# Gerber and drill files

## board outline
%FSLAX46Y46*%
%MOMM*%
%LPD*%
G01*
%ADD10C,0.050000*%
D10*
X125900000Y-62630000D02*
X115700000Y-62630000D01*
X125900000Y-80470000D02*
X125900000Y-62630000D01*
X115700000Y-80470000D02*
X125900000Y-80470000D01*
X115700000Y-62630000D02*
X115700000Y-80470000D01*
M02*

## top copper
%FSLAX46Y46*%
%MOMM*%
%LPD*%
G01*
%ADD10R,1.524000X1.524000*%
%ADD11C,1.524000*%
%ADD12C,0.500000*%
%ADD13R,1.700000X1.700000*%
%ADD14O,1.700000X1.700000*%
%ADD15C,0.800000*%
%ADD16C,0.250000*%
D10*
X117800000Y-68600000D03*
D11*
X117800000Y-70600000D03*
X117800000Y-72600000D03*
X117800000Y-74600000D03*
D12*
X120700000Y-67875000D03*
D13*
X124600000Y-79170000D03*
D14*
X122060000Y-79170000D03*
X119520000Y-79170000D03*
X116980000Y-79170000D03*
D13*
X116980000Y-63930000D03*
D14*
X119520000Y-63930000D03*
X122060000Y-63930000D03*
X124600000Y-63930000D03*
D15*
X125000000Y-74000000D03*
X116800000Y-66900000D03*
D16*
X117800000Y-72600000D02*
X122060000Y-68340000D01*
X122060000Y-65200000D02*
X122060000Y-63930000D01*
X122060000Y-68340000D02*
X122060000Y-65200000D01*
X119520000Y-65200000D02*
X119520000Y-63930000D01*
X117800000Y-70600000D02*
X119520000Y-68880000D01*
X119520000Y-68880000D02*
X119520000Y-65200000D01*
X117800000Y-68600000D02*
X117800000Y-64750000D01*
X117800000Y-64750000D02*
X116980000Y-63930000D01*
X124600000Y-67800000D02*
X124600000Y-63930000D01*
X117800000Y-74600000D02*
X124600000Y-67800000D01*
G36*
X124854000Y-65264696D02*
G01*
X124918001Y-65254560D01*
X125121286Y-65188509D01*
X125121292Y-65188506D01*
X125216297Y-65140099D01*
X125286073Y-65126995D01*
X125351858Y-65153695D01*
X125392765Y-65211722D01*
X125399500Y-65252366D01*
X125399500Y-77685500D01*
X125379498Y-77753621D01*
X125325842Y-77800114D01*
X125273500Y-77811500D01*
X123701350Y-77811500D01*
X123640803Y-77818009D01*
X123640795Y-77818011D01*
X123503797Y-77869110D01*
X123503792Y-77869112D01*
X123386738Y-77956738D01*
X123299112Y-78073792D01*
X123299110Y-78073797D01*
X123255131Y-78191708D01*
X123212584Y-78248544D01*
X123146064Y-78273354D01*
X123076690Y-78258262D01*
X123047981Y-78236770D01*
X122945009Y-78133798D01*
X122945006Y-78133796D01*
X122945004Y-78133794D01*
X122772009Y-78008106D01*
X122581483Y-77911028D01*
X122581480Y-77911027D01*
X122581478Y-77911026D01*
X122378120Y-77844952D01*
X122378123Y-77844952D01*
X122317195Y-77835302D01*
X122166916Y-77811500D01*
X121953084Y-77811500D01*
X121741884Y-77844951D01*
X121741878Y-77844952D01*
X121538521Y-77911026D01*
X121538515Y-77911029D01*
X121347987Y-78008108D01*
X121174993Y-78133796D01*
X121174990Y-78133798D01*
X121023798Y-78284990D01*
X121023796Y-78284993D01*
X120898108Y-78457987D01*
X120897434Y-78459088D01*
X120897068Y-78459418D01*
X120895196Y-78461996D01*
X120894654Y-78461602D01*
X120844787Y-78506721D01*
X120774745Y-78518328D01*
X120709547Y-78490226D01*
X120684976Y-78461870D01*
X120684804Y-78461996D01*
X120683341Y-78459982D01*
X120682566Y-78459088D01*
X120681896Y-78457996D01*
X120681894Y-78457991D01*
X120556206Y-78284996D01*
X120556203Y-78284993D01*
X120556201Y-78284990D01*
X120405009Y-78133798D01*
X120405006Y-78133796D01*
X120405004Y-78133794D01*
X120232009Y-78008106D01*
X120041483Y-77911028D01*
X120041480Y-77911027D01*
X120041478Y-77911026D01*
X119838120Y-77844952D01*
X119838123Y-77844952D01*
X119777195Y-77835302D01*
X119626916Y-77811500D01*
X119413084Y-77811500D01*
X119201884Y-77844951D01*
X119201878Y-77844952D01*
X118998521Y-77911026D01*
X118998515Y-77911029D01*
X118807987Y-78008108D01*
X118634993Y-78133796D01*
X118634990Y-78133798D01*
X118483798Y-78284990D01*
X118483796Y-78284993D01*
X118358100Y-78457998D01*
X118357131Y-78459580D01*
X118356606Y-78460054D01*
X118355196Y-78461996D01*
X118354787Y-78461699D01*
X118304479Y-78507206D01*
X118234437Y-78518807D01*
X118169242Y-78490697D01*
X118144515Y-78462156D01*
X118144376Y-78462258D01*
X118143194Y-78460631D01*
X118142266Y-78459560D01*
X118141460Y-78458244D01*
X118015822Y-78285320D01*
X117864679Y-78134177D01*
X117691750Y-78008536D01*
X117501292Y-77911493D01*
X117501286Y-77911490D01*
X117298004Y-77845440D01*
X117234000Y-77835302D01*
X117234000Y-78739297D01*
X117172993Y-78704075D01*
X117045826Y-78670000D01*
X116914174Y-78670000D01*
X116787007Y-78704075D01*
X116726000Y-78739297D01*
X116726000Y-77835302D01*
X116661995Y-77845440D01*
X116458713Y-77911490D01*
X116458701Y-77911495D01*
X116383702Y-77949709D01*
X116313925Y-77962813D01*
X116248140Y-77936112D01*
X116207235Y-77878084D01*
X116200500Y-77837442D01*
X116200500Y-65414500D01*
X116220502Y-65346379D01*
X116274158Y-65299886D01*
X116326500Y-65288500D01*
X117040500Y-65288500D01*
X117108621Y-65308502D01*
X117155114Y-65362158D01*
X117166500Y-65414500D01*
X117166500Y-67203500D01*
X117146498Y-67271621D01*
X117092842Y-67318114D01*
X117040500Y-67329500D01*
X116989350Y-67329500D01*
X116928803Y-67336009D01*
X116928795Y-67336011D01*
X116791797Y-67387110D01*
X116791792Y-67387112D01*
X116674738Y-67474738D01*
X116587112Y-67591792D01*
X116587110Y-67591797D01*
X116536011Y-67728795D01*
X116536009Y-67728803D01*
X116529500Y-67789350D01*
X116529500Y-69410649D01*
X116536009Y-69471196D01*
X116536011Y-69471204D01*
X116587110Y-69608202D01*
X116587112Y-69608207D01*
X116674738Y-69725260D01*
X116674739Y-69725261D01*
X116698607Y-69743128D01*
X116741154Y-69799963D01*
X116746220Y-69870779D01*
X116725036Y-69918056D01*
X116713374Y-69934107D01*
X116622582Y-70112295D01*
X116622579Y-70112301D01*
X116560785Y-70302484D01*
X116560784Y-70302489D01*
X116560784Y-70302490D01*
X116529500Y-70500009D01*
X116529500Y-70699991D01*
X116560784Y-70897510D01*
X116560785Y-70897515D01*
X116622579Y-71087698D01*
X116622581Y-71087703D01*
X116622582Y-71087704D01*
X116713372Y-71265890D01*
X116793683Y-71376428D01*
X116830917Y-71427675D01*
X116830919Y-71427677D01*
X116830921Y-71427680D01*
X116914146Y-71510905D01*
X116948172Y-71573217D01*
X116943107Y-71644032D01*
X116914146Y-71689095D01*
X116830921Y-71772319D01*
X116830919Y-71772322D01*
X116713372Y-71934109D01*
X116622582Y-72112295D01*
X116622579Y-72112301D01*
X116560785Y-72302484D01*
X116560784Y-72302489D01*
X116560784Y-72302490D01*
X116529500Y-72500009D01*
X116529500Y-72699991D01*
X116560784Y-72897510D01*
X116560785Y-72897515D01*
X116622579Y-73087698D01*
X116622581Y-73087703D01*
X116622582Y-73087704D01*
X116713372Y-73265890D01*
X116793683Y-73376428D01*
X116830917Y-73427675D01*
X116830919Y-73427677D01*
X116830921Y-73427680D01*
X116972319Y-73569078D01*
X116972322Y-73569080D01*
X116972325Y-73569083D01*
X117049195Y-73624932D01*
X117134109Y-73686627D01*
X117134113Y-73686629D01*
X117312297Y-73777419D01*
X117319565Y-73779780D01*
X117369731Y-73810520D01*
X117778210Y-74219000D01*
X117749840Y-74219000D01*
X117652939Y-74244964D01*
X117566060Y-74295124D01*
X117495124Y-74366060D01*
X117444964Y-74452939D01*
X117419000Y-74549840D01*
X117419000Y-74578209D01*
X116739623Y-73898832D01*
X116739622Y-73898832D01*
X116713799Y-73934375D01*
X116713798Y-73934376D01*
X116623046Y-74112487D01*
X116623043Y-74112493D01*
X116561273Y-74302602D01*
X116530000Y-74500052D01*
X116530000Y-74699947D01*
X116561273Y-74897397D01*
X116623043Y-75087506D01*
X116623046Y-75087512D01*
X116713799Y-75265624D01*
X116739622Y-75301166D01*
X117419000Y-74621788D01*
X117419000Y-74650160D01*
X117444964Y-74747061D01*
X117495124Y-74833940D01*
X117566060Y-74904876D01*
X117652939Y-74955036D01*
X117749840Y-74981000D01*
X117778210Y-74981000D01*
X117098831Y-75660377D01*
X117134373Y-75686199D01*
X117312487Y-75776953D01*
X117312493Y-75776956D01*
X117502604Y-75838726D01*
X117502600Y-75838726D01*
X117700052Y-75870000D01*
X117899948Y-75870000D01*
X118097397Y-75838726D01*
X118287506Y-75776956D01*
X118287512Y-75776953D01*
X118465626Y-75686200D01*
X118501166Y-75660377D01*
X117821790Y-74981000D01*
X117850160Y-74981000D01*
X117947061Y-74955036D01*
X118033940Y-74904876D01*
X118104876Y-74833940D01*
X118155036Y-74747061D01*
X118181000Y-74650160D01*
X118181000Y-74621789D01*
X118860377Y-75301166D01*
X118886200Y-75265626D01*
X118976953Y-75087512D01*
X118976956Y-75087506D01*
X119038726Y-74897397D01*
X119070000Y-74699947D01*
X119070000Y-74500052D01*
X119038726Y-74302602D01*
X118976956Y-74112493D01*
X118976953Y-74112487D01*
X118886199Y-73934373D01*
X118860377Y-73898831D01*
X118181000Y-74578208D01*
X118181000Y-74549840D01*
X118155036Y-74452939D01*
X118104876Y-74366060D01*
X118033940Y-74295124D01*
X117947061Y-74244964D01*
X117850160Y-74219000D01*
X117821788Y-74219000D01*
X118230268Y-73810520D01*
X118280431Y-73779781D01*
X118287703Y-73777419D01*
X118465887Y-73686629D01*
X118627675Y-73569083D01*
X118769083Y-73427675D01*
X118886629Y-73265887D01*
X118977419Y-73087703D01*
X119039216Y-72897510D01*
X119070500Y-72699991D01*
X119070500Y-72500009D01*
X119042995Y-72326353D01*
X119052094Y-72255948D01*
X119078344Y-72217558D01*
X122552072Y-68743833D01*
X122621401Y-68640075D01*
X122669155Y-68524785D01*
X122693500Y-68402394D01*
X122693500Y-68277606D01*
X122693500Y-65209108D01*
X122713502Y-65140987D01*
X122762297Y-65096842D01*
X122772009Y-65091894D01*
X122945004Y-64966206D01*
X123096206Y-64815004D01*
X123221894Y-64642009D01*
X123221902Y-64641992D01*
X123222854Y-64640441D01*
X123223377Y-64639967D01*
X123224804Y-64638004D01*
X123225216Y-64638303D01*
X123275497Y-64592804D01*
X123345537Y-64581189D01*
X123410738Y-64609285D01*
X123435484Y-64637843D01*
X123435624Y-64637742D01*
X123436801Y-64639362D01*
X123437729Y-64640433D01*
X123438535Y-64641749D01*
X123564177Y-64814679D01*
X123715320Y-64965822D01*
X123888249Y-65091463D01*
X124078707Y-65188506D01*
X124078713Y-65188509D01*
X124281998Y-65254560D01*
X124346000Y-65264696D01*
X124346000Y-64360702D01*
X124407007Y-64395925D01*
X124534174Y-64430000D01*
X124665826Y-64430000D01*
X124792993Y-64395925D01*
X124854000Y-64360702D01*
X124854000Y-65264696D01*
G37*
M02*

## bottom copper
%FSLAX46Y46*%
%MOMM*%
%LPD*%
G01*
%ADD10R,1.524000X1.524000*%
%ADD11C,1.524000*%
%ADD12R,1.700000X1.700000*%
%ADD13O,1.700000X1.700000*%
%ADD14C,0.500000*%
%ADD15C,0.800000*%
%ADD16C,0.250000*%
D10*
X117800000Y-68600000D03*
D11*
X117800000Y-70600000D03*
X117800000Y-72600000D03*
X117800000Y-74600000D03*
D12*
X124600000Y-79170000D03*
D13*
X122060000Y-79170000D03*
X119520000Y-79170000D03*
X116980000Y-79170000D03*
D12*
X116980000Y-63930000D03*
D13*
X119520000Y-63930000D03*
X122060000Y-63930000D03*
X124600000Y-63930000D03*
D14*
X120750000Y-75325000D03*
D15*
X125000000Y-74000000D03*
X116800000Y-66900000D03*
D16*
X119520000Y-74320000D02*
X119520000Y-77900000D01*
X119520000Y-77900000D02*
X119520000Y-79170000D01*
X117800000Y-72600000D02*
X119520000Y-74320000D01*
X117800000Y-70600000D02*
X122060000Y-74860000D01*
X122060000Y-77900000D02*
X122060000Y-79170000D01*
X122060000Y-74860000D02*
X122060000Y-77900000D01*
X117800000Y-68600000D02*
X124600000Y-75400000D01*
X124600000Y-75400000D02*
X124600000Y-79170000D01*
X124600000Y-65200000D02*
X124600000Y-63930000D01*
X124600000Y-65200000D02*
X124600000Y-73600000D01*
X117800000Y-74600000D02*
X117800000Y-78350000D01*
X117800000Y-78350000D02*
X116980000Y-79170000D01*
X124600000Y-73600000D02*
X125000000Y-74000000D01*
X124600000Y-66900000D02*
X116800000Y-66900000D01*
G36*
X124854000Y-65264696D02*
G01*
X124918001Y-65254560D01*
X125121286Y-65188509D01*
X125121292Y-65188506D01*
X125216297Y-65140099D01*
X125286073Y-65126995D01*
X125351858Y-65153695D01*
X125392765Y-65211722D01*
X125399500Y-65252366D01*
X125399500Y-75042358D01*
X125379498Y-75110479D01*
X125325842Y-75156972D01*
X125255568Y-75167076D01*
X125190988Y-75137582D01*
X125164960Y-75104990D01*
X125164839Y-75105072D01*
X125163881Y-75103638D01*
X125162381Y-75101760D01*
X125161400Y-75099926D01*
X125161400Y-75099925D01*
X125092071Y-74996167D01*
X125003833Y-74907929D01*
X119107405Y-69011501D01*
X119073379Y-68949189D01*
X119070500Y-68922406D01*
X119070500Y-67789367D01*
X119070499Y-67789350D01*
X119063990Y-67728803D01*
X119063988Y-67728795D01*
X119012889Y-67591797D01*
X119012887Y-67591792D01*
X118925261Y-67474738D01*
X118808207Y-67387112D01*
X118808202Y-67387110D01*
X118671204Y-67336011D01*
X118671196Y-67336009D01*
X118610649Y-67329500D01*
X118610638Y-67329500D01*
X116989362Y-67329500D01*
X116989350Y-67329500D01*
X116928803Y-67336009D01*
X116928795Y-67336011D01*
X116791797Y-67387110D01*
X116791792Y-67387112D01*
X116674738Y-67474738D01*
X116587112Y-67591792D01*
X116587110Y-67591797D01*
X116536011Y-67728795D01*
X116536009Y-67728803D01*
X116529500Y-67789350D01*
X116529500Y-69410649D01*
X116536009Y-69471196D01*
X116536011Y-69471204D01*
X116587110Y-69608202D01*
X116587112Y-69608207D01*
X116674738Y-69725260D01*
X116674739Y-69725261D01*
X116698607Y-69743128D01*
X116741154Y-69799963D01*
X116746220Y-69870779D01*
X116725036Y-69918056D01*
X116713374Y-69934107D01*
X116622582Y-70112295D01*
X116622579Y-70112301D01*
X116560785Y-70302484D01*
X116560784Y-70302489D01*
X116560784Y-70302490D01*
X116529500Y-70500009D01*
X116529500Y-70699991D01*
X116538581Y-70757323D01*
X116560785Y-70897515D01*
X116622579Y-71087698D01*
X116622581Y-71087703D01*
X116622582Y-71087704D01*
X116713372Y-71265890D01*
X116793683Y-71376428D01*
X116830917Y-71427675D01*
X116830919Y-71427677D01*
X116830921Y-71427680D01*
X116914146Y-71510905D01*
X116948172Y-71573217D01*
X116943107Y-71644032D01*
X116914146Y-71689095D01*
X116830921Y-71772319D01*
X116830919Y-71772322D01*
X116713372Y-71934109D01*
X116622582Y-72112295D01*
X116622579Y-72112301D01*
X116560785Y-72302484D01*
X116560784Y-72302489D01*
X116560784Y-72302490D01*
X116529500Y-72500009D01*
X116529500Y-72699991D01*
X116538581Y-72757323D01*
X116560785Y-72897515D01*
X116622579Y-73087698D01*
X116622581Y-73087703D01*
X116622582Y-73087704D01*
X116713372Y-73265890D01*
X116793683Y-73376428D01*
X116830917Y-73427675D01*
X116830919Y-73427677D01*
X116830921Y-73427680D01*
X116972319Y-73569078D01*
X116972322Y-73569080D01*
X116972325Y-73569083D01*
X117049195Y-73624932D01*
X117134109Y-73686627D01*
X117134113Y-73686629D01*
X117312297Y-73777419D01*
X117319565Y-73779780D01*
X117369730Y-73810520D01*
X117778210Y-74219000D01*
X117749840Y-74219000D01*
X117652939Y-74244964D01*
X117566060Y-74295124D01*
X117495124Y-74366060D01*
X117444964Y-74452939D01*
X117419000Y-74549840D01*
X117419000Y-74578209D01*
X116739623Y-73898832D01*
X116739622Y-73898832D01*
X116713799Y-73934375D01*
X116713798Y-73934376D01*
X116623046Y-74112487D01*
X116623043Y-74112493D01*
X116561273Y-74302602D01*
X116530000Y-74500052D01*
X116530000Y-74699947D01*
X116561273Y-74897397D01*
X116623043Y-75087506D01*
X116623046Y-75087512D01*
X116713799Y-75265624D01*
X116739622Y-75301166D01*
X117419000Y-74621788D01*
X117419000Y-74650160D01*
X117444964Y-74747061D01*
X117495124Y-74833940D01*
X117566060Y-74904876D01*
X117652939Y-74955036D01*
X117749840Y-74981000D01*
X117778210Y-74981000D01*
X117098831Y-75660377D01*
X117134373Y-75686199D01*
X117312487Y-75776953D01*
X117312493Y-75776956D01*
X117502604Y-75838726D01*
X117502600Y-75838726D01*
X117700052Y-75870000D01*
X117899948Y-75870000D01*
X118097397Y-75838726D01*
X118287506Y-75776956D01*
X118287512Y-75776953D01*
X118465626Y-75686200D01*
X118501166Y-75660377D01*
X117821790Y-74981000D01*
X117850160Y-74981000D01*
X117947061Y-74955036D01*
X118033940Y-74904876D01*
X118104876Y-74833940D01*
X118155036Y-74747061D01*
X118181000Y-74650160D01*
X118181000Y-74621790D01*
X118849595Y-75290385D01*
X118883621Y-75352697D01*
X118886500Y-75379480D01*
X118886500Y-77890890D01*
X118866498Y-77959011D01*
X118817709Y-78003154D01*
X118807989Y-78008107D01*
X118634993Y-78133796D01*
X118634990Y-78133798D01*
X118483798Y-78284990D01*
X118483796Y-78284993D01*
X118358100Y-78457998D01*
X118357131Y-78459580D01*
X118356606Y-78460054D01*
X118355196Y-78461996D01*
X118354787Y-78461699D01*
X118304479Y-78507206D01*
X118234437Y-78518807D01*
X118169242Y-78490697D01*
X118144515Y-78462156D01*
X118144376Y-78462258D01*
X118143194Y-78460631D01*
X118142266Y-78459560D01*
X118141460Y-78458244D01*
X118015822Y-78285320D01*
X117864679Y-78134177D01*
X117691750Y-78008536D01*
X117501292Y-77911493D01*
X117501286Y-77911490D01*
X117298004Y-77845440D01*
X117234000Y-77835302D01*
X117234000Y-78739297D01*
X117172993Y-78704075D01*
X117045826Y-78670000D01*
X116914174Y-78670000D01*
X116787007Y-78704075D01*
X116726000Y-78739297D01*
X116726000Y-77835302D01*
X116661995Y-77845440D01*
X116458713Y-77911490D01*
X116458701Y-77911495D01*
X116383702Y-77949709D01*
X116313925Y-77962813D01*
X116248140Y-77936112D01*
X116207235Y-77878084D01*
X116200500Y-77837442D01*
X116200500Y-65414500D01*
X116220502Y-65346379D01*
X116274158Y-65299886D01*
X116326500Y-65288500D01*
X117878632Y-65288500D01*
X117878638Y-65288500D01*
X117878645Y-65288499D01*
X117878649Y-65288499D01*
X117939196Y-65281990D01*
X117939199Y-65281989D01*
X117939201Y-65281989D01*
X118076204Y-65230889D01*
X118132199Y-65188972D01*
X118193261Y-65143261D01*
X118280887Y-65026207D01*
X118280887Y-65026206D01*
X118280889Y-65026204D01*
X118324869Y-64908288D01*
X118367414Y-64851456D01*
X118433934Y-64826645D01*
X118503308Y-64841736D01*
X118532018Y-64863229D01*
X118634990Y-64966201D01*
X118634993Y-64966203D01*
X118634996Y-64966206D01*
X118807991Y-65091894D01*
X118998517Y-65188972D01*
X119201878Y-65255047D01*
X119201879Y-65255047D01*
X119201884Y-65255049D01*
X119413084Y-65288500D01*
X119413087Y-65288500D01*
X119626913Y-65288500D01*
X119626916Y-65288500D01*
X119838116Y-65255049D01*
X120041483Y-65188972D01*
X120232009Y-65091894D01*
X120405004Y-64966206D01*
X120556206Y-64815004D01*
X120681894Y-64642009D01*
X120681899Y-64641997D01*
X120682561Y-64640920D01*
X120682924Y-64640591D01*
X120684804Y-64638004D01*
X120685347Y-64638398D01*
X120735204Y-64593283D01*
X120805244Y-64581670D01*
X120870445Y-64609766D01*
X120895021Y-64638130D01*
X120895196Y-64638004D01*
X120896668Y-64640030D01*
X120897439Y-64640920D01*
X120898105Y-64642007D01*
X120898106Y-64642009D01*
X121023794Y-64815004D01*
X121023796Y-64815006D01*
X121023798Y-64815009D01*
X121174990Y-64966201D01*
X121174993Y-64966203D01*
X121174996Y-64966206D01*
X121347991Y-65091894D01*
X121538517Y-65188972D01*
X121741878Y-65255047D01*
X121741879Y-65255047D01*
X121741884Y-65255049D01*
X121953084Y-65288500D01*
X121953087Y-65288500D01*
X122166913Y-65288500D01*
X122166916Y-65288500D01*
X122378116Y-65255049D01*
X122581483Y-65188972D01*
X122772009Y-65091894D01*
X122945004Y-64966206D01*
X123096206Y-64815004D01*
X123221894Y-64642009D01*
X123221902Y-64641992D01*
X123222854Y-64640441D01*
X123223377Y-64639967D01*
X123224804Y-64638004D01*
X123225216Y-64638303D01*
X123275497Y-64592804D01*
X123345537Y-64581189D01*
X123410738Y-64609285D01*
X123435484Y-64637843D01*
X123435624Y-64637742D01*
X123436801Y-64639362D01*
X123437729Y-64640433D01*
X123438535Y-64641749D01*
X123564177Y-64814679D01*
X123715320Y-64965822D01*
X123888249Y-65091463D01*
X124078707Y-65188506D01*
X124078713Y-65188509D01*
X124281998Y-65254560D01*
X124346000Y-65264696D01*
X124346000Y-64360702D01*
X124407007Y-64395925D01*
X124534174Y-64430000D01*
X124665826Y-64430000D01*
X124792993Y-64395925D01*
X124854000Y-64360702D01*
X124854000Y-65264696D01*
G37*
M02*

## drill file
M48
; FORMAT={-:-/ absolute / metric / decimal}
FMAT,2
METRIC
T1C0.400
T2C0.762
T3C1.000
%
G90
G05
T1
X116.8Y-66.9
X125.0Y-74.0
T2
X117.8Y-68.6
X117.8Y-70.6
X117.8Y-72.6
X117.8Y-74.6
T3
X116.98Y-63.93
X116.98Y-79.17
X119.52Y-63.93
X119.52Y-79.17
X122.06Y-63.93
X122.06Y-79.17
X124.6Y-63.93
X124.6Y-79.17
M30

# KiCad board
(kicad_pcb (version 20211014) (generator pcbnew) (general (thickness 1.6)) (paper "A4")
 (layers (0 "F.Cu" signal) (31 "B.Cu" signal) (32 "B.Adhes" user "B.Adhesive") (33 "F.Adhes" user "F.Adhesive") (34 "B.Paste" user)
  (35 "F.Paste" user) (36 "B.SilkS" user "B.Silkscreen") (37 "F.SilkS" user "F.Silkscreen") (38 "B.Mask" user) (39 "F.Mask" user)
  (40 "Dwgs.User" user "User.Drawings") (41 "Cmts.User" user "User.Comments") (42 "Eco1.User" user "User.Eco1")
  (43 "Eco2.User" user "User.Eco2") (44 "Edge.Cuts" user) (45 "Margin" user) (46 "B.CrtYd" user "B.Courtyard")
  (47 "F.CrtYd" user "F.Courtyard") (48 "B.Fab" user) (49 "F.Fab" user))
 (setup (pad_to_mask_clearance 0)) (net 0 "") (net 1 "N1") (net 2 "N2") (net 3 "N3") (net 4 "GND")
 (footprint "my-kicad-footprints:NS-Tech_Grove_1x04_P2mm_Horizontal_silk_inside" (layer "F.Cu") (at 117.8 71.6)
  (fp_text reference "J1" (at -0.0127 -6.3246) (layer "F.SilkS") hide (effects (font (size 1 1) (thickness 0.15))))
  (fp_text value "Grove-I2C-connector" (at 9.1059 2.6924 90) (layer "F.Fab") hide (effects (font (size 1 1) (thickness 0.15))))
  (pad "1" thru_hole rect locked (at 0 -3) (size 1.524 1.524) (drill 0.762) (layers *.Cu *.Mask) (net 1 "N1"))
  (pad "2" thru_hole circle locked (at 0 -1) (size 1.524 1.524) (drill 0.762) (layers *.Cu *.Mask) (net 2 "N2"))
  (pad "3" thru_hole circle locked (at 0 1) (size 1.524 1.524) (drill 0.762) (layers *.Cu *.Mask) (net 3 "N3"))
  (pad "4" thru_hole circle locked (at 0 3) (size 1.524 1.524) (drill 0.762) (layers *.Cu *.Mask) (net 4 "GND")))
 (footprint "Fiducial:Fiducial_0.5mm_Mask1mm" (layer "F.Cu") (at 120.7 67.875)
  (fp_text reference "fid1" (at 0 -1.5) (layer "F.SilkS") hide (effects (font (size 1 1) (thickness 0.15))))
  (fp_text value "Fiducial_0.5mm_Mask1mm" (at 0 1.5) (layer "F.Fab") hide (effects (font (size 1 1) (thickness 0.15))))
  (pad "" smd circle locked (at 0 0) (size 0.5 0.5) (layers "F.Cu" "F.Mask") (solder_mask_margin 0.25) (clearance 0.25)))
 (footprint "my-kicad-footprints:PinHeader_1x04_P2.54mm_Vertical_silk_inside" (layer "B.Cu") (at 124.6 79.17 90)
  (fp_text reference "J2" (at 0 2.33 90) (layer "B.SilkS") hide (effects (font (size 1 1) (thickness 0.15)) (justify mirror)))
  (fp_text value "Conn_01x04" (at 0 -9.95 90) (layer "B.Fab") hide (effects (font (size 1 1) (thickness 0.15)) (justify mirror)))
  (pad "1" thru_hole rect locked (at 0 0 90) (size 1.7 1.7) (drill 1) (layers *.Cu *.Mask) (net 1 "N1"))
  (pad "2" thru_hole oval locked (at 0 -2.54 90) (size 1.7 1.7) (drill 1) (layers *.Cu *.Mask) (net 2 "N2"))
  (pad "3" thru_hole oval locked (at 0 -5.08 90) (size 1.7 1.7) (drill 1) (layers *.Cu *.Mask) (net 3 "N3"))
  (pad "4" thru_hole oval locked (at 0 -7.62 90) (size 1.7 1.7) (drill 1) (layers *.Cu *.Mask) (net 4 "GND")))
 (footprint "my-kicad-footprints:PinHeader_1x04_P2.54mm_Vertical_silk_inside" (layer "B.Cu") (at 116.98 63.93 -90)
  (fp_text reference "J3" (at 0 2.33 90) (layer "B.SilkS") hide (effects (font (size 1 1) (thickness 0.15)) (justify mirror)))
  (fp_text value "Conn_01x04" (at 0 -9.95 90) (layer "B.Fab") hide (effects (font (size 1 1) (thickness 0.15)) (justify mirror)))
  (pad "1" thru_hole rect locked (at 0 0 270) (size 1.7 1.7) (drill 1) (layers *.Cu *.Mask) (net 1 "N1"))
  (pad "2" thru_hole oval locked (at 0 -2.54 270) (size 1.7 1.7) (drill 1) (layers *.Cu *.Mask) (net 2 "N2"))
  (pad "3" thru_hole oval locked (at 0 -5.08 270) (size 1.7 1.7) (drill 1) (layers *.Cu *.Mask) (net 3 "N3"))
  (pad "4" thru_hole oval locked (at 0 -7.62 270) (size 1.7 1.7) (drill 1) (layers *.Cu *.Mask) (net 4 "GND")))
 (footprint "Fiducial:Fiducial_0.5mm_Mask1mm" (layer "B.Cu") (at 120.75 75.325)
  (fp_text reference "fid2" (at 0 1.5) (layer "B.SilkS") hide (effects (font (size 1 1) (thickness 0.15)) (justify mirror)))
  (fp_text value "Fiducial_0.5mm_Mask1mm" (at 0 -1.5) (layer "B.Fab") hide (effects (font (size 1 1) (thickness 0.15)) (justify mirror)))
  (pad "" smd circle locked (at 0 0) (size 0.5 0.5) (layers "B.Cu" "B.Mask") (solder_mask_margin 0.25) (clearance 0.25)))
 (gr_line (start 125.9 62.63) (end 115.7 62.63) (layer "Edge.Cuts") (width 0.05))
 (gr_line (start 125.9 80.47) (end 125.9 62.63) (layer "Edge.Cuts") (width 0.05))
 (gr_line (start 115.7 80.47) (end 125.9 80.47) (layer "Edge.Cuts") (width 0.05))
 (gr_line (start 115.7 62.63) (end 115.7 80.47) (layer "Edge.Cuts") (width 0.05))
 (segment (start 117.8 72.6) (end 122.06 68.34) (width 0.25) (layer "F.Cu") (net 3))
 (segment (start 122.06 65.2) (end 122.06 63.93) (width 0.25) (layer "F.Cu") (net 3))
 (segment (start 122.06 68.34) (end 122.06 65.2) (width 0.25) (layer "F.Cu") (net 3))
 (segment (start 119.52 74.32) (end 119.52 77.9) (width 0.25) (layer "B.Cu") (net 3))
 (segment (start 119.52 77.9) (end 119.52 79.17) (width 0.25) (layer "B.Cu") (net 3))
 (segment (start 117.8 72.6) (end 119.52 74.32) (width 0.25) (layer "B.Cu") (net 3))
 (segment (start 119.52 65.2) (end 119.52 63.93) (width 0.25) (layer "F.Cu") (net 2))
 (segment (start 117.8 70.6) (end 119.52 68.88) (width 0.25) (layer "F.Cu") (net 2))
 (segment (start 119.52 68.88) (end 119.52 65.2) (width 0.25) (layer "F.Cu") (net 2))
 (segment (start 117.8 70.6) (end 122.06 74.86) (width 0.25) (layer "B.Cu") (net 2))
 (segment (start 122.06 77.9) (end 122.06 79.17) (width 0.25) (layer "B.Cu") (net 2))
 (segment (start 122.06 74.86) (end 122.06 77.9) (width 0.25) (layer "B.Cu") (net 2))
 (segment (start 117.8 68.6) (end 117.8 64.75) (width 0.25) (layer "F.Cu") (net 1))
 (segment (start 117.8 64.75) (end 116.98 63.93) (width 0.25) (layer "F.Cu") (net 1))
 (segment (start 117.8 68.6) (end 124.6 75.4) (width 0.25) (layer "B.Cu") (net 1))
 (segment (start 124.6 75.4) (end 124.6 79.17) (width 0.25) (layer "B.Cu") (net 1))
 (segment (start 124.6 67.8) (end 124.6 63.93) (width 0.25) (layer "F.Cu") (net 4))
 (segment (start 117.8 74.6) (end 124.6 67.8) (width 0.25) (layer "F.Cu") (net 4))
 (via (at 125 74) (size 0.8) (drill 0.4) (layers "F.Cu" "B.Cu") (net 4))
 (via (at 116.8 66.9) (size 0.8) (drill 0.4) (layers "F.Cu" "B.Cu") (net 4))
 (segment (start 124.6 65.2) (end 124.6 63.93) (width 0.25) (layer "B.Cu") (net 4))
 (segment (start 124.6 65.2) (end 124.6 73.6) (width 0.25) (layer "B.Cu") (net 4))
 (segment (start 117.8 74.6) (end 117.8 78.35) (width 0.25) (layer "B.Cu") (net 4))
 (segment (start 117.8 78.35) (end 116.98 79.17) (width 0.25) (layer "B.Cu") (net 4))
 (segment (start 124.6 73.6) (end 125 74) (width 0.25) (layer "B.Cu") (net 4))
 (segment (start 124.6 66.9) (end 116.8 66.9) (width 0.25) (layer "B.Cu") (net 4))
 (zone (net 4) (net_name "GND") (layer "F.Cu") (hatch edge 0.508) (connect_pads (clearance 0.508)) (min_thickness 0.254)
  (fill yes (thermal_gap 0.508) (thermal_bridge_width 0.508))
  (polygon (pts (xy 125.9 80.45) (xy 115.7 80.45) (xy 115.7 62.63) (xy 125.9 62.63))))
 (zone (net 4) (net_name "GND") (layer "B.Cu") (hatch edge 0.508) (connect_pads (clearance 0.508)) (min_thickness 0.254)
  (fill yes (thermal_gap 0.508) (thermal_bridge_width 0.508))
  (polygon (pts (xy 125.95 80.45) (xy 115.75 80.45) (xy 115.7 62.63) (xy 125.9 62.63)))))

